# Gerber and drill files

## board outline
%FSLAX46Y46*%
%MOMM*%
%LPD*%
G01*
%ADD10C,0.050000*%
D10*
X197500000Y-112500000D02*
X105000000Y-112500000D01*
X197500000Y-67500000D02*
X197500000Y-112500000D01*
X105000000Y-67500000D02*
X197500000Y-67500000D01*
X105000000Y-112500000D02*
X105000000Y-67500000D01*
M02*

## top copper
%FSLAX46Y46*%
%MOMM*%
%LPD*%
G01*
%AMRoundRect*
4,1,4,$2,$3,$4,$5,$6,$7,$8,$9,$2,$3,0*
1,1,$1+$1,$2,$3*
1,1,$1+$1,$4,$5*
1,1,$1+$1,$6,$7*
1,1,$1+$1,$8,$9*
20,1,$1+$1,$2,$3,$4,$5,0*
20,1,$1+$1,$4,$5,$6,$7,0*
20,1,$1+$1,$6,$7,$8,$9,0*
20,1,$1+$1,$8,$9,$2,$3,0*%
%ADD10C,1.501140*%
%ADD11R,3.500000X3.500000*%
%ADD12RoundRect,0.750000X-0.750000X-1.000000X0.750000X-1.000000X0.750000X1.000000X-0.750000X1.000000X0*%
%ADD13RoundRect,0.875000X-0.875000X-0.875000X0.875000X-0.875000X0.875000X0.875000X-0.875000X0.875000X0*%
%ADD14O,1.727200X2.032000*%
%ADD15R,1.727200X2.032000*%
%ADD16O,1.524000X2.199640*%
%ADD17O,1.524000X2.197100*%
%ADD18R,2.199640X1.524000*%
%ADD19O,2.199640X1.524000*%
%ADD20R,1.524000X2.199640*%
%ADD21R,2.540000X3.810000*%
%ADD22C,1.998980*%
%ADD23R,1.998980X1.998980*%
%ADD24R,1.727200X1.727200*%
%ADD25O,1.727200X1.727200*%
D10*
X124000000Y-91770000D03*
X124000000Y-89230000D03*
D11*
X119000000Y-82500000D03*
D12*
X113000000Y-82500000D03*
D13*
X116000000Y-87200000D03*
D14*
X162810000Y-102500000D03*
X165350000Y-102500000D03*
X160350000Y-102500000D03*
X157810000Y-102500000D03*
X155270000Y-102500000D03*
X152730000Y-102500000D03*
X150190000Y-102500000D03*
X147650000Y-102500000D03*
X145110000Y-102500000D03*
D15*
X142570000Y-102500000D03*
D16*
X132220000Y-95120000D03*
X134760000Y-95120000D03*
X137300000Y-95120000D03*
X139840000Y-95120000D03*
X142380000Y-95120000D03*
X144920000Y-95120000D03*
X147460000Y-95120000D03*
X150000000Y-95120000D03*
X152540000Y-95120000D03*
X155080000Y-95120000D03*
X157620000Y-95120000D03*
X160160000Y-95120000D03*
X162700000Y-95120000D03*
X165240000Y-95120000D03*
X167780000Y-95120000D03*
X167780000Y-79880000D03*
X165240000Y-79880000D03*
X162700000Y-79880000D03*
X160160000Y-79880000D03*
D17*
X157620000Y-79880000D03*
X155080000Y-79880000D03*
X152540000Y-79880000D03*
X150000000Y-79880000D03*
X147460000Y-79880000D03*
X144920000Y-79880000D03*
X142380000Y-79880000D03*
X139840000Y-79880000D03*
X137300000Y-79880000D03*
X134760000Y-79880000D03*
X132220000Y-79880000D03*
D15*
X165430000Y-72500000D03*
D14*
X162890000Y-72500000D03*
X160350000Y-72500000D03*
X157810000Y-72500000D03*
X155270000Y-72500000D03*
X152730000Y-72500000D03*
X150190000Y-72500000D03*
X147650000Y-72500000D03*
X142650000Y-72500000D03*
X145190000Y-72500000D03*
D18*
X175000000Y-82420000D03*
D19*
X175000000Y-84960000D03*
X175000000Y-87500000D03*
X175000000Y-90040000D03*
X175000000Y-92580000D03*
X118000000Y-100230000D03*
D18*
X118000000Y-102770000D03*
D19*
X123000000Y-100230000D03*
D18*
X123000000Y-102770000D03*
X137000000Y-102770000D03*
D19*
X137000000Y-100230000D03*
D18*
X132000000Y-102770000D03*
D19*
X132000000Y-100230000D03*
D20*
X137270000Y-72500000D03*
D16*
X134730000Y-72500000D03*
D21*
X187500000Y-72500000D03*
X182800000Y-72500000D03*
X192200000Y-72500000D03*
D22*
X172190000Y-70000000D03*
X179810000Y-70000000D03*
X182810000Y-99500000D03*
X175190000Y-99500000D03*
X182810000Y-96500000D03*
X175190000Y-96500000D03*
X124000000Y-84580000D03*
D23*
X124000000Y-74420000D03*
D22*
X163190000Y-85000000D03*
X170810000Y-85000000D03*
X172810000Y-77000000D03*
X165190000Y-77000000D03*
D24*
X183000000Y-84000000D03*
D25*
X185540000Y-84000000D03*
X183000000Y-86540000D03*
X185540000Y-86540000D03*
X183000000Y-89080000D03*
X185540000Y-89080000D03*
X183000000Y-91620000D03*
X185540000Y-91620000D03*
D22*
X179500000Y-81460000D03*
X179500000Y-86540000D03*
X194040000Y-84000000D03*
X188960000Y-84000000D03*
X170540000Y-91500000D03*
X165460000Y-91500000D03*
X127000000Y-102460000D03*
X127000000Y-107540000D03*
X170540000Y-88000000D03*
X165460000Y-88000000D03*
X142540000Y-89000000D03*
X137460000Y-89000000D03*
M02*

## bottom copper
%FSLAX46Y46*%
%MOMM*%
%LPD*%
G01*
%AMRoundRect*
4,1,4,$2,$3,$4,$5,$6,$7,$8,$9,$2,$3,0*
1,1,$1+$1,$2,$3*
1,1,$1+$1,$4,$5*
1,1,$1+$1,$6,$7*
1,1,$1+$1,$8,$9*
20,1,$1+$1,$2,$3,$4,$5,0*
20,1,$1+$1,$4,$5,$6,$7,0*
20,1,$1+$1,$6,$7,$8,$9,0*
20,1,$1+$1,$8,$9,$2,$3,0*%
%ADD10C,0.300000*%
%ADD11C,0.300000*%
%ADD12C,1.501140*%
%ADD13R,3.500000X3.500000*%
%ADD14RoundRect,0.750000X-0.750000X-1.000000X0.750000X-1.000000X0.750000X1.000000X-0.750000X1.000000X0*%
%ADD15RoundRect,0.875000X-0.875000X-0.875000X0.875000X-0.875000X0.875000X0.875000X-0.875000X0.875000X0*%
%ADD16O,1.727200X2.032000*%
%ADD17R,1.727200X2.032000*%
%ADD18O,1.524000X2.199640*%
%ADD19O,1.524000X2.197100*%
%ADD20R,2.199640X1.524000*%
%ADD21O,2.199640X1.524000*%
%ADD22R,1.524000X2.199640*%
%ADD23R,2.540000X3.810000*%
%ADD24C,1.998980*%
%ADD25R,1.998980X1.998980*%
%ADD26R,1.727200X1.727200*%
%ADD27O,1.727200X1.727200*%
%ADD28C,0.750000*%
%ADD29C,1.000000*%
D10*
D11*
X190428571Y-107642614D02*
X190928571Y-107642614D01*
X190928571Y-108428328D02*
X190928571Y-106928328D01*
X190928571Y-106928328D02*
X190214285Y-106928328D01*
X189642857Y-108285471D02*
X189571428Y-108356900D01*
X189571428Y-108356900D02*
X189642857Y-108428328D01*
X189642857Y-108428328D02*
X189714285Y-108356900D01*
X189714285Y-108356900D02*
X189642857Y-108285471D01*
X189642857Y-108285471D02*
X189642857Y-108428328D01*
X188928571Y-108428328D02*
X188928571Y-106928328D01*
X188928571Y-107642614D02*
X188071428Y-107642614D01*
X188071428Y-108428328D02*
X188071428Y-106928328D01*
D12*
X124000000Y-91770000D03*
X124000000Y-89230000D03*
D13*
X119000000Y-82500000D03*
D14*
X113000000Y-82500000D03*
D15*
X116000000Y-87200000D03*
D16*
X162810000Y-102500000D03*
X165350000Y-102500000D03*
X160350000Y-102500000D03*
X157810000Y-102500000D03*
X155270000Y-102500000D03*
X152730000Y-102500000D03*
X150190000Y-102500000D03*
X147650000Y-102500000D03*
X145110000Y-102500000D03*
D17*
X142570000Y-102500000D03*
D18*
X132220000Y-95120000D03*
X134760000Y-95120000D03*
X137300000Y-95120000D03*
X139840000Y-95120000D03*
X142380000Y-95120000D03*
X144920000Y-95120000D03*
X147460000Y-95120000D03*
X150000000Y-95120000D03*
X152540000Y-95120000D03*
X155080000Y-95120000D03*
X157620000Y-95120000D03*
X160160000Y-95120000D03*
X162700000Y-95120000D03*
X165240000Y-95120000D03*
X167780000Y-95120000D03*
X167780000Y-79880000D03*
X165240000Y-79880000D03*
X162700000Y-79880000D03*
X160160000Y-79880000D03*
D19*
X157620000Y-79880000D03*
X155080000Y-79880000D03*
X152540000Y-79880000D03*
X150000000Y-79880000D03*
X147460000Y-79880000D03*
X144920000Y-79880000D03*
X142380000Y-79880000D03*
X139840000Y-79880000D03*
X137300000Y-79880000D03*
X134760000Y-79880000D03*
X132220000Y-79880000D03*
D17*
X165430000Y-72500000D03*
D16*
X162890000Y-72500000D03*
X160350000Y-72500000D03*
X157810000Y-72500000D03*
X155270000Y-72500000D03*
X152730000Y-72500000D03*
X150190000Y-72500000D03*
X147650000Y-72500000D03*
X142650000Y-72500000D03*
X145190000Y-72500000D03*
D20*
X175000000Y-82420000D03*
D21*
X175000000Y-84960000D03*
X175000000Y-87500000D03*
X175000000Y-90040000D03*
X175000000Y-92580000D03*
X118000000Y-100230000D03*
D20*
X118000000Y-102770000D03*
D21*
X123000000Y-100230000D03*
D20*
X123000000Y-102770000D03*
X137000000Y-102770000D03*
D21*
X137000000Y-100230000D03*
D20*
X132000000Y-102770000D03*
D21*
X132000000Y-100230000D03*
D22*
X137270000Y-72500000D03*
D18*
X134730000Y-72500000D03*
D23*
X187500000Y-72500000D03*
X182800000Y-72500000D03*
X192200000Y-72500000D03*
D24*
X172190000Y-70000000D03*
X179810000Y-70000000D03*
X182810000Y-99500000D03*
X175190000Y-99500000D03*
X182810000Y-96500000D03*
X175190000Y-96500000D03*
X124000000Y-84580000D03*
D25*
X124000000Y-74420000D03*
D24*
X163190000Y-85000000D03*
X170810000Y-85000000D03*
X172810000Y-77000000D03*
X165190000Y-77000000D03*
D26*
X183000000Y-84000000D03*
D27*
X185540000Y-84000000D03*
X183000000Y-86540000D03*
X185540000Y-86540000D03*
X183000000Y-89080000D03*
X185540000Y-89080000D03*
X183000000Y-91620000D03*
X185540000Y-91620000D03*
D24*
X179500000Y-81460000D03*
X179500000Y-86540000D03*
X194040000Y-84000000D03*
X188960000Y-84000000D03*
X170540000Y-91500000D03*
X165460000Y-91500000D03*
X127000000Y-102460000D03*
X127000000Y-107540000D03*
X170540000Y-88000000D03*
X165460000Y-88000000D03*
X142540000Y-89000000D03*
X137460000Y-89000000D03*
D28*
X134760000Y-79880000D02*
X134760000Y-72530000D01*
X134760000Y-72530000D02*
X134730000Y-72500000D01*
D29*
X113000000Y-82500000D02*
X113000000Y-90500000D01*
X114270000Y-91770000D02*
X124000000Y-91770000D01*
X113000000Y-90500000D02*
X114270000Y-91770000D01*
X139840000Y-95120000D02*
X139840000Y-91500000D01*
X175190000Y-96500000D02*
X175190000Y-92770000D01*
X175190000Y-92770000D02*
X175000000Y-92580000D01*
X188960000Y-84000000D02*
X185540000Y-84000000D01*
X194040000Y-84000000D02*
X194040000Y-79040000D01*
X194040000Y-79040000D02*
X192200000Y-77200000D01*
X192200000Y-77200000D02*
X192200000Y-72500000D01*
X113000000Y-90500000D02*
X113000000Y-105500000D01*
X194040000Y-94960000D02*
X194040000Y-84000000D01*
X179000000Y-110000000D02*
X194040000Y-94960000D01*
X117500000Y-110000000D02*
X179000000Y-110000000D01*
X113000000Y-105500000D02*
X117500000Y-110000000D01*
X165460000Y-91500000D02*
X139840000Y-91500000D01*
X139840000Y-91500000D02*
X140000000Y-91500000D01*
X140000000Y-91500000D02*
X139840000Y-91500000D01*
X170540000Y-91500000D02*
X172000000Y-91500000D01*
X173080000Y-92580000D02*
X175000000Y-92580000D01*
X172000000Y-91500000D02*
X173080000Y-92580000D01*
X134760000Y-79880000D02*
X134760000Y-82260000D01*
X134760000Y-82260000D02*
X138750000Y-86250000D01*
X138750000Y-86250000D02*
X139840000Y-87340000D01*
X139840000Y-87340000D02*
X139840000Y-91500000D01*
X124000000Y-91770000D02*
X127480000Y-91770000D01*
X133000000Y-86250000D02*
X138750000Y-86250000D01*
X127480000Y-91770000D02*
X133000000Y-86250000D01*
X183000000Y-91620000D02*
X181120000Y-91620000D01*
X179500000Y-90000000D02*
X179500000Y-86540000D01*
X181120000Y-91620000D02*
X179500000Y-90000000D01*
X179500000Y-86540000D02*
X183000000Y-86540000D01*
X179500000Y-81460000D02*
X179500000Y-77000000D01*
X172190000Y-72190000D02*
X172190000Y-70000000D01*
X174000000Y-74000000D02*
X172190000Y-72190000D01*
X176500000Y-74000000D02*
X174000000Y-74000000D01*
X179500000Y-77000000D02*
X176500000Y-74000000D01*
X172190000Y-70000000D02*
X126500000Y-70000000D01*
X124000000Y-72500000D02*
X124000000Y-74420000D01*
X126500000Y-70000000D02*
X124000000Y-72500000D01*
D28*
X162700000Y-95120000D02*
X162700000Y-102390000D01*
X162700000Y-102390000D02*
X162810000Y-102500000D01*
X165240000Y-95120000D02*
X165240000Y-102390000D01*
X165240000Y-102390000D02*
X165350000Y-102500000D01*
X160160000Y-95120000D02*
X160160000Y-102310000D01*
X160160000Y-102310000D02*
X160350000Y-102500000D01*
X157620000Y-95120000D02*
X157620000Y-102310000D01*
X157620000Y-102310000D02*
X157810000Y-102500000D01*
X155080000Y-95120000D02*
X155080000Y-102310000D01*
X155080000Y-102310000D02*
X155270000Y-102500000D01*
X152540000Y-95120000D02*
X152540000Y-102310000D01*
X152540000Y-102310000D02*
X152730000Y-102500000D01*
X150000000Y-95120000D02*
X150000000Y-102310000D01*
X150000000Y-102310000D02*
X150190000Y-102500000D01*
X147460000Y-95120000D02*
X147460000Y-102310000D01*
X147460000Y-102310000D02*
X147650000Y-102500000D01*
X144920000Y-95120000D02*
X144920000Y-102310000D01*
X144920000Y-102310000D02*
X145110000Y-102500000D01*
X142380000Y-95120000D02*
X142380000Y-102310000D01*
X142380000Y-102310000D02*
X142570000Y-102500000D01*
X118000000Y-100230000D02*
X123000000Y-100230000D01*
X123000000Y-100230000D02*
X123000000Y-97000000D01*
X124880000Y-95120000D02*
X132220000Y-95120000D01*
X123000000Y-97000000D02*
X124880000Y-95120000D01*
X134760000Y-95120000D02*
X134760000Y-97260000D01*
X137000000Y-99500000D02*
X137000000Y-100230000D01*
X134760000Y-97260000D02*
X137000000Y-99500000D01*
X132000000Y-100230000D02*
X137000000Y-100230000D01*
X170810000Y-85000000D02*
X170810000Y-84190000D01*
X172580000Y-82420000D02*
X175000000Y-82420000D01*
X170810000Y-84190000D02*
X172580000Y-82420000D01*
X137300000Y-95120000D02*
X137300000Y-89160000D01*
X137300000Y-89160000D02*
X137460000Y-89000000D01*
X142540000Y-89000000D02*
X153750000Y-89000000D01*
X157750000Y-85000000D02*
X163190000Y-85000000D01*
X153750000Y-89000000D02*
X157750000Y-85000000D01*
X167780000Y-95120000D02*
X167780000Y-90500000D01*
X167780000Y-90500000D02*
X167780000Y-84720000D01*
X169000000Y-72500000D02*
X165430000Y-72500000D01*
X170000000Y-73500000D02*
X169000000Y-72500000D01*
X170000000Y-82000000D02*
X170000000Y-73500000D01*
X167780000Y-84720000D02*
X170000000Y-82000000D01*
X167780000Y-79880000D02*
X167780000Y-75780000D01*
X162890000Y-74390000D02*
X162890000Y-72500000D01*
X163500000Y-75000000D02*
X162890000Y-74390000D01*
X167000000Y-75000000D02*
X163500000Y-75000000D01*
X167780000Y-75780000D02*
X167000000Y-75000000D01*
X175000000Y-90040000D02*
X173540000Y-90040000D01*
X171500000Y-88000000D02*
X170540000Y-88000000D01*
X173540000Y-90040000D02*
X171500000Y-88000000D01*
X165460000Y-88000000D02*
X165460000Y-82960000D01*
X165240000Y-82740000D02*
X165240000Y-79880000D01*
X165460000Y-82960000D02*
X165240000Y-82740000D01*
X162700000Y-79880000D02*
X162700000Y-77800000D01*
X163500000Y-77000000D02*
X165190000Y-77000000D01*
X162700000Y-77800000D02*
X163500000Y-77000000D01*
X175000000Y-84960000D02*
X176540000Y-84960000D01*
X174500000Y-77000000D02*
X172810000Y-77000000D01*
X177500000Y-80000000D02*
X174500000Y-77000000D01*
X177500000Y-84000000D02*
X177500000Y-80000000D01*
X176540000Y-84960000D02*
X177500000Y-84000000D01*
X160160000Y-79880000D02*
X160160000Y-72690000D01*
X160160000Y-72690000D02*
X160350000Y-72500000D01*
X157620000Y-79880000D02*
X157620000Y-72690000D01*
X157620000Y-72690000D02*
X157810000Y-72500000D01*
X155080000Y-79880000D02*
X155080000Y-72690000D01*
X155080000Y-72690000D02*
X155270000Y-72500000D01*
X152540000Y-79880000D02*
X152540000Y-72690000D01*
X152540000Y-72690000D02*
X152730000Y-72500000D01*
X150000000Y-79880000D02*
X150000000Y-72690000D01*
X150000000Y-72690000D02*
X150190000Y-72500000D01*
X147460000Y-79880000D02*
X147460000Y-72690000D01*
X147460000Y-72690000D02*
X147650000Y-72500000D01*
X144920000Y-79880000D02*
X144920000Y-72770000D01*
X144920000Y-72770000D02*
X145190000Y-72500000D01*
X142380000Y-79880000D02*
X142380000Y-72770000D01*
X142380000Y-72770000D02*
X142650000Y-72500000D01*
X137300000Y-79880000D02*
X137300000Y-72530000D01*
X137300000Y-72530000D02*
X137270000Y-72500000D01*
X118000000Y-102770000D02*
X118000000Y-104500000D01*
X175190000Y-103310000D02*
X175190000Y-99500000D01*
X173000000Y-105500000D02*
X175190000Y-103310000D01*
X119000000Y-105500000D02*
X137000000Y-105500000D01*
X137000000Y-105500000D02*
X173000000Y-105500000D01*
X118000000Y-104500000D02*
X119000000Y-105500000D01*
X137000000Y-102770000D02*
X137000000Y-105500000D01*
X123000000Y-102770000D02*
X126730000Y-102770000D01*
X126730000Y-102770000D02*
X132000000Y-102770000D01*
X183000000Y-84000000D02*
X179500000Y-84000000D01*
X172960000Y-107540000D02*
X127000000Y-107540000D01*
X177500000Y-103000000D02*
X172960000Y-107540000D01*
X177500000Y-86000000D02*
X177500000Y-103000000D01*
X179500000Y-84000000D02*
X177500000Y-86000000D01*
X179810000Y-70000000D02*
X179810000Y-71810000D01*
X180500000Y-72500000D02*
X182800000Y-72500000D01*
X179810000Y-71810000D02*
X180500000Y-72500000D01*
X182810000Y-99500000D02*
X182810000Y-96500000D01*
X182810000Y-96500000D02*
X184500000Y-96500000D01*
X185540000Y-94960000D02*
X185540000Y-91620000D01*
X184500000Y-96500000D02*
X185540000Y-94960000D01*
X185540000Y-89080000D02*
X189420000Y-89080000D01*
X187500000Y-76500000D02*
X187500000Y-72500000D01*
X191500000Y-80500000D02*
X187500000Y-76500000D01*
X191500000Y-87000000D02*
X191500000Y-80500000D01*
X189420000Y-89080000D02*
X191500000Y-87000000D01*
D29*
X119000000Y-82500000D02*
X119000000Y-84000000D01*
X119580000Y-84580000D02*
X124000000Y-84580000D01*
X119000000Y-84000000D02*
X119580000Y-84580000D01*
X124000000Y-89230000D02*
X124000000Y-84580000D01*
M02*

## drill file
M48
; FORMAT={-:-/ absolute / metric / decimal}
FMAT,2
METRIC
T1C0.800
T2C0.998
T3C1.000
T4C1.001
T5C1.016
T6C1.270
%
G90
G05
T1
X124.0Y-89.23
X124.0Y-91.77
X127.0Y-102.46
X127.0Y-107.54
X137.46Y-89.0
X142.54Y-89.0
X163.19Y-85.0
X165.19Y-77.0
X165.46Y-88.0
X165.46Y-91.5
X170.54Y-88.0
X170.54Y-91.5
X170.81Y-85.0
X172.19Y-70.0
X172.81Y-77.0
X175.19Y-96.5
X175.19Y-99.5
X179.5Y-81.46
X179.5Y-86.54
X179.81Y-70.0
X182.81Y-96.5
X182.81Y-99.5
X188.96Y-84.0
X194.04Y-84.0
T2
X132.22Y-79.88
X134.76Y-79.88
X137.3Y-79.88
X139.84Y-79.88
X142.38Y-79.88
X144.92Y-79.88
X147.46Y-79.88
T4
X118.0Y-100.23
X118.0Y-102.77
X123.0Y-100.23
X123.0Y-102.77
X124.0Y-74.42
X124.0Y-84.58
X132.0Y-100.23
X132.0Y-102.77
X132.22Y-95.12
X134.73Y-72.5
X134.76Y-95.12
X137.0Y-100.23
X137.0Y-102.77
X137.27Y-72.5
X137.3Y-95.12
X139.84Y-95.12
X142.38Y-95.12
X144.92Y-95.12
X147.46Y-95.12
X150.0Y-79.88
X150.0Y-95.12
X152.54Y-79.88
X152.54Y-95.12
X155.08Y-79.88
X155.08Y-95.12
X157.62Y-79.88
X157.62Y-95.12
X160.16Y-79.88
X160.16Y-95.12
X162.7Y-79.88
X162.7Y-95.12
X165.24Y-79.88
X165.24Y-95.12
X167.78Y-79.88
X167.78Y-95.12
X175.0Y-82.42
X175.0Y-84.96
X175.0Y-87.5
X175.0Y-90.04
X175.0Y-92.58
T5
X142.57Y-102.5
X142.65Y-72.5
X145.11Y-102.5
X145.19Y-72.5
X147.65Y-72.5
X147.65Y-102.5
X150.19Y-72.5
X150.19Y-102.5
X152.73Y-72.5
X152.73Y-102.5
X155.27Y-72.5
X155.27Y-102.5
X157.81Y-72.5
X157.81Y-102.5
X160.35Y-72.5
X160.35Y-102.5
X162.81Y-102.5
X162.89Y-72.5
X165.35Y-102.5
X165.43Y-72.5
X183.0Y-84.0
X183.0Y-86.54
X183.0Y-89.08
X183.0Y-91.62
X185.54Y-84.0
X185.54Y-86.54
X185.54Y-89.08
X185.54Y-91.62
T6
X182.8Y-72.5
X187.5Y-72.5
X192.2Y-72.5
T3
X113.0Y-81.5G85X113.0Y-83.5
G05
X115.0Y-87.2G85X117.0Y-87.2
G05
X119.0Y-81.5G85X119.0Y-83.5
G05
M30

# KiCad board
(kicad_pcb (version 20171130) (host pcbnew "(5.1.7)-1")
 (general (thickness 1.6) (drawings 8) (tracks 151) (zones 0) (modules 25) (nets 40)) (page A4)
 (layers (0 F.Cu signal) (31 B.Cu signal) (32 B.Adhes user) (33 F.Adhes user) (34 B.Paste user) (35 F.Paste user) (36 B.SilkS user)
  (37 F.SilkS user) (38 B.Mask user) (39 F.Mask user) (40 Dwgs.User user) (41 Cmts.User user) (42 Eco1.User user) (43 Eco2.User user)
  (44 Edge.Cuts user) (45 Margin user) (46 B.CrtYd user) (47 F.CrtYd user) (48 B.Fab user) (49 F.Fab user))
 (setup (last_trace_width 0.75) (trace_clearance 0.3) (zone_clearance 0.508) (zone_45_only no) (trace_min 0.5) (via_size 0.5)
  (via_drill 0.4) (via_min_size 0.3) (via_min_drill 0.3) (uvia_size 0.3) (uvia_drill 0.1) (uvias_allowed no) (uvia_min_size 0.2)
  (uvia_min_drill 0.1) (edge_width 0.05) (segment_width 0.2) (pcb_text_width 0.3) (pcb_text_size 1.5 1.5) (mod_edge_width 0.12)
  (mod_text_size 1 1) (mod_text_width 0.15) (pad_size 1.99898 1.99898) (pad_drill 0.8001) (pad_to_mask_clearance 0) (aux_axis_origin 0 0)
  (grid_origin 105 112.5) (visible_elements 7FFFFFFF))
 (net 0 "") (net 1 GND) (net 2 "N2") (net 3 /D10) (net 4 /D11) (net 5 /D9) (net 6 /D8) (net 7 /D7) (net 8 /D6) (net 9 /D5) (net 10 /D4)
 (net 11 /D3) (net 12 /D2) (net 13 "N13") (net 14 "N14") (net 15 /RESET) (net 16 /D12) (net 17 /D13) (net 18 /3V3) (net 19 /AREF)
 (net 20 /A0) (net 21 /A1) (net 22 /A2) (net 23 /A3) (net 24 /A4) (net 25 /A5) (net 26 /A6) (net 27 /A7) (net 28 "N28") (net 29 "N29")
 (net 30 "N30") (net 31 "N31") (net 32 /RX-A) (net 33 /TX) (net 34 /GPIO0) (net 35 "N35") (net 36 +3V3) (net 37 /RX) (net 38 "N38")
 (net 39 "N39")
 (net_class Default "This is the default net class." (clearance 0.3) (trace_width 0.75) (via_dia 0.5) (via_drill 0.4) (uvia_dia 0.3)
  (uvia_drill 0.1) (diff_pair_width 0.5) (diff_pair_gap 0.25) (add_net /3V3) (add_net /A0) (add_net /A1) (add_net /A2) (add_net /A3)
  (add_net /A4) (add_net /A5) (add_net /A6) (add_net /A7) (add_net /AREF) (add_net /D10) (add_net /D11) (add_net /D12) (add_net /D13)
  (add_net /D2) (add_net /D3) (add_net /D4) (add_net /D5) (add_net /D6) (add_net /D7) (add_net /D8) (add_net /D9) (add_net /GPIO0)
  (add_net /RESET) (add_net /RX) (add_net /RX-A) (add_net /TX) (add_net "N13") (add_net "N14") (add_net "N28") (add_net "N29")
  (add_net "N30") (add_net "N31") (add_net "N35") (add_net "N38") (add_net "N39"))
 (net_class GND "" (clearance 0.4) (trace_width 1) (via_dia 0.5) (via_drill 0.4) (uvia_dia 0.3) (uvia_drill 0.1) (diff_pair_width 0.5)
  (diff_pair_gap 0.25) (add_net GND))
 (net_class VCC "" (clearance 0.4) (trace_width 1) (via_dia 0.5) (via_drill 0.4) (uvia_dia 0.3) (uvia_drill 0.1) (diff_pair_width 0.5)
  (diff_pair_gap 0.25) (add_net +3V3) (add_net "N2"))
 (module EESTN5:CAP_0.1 (layer F.Cu) (at 124 90.5 90)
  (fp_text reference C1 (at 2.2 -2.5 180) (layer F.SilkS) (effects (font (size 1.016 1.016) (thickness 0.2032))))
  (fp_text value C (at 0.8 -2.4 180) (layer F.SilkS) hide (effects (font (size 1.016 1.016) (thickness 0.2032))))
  (pad 1 thru_hole circle (at -1.27 0 90) (size 1.50114 1.50114) (drill 0.8001) (layers *.Cu *.Mask F.SilkS) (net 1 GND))
  (pad 2 thru_hole circle (at 1.27 0 90) (size 1.50114 1.50114) (drill 0.8001) (layers *.Cu *.Mask F.SilkS) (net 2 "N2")))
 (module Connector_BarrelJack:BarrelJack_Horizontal (layer F.Cu) (at 119 82.5)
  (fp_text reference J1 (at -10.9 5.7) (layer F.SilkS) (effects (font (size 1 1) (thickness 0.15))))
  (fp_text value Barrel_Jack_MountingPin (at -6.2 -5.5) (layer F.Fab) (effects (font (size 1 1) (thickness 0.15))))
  (pad 1 thru_hole rect (at 0 0) (size 3.5 3.5) (drill oval 1 3) (layers *.Cu *.Mask) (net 2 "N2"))
  (pad 2 thru_hole roundrect (at -6 0) (size 3 3.5) (drill oval 1 3) (layers *.Cu *.Mask) (roundrect_rratio 0.25) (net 1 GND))
  (pad 3 thru_hole roundrect (at -3 4.7) (size 3.5 3.5) (drill oval 3 1) (layers *.Cu *.Mask) (roundrect_rratio 0.25)))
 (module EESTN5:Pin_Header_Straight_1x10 (layer F.Cu) (at 154 102.5 90)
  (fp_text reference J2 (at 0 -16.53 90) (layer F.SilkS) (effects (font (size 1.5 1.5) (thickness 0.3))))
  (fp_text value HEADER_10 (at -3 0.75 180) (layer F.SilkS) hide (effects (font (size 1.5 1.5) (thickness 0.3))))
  (pad 9 thru_hole oval (at 0 8.81 90) (size 2.032 1.7272) (drill 1.016) (layers *.Cu *.Mask F.SilkS) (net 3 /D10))
  (pad 10 thru_hole oval (at 0 11.35 90) (size 2.032 1.7272) (drill 1.016) (layers *.Cu *.Mask F.SilkS) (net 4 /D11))
  (pad 8 thru_hole oval (at 0 6.35 90) (size 2.032 1.7272) (drill 1.016) (layers *.Cu *.Mask F.SilkS) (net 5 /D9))
  (pad 7 thru_hole oval (at 0 3.81 90) (size 2.032 1.7272) (drill 1.016) (layers *.Cu *.Mask F.SilkS) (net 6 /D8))
  (pad 6 thru_hole oval (at 0 1.27 90) (size 2.032 1.7272) (drill 1.016) (layers *.Cu *.Mask F.SilkS) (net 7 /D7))
  (pad 5 thru_hole oval (at 0 -1.27 90) (size 2.032 1.7272) (drill 1.016) (layers *.Cu *.Mask F.SilkS) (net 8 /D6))
  (pad 4 thru_hole oval (at 0 -3.81 90) (size 2.032 1.7272) (drill 1.016) (layers *.Cu *.Mask F.SilkS) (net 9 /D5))
  (pad 3 thru_hole oval (at 0 -6.35 90) (size 2.032 1.7272) (drill 1.016) (layers *.Cu *.Mask F.SilkS) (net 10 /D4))
  (pad 2 thru_hole oval (at 0 -8.89 90) (size 2.032 1.7272) (drill 1.016) (layers *.Cu *.Mask F.SilkS) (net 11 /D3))
  (pad 1 thru_hole rect (at 0 -11.43 90) (size 2.032 1.7272) (drill 1.016) (layers *.Cu *.Mask F.SilkS) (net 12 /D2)))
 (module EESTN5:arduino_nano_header (layer F.Cu) (at 150 87.5)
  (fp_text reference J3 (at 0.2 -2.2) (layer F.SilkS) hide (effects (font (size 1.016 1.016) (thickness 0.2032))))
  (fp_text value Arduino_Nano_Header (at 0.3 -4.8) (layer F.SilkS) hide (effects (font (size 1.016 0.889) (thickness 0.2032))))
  (pad 1 thru_hole oval (at -17.78 7.62) (size 1.524 2.19964) (drill 1.00076) (layers *.Cu *.Mask F.SilkS) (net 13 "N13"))
  (pad 2 thru_hole oval (at -15.24 7.62) (size 1.524 2.19964) (drill 1.00076) (layers *.Cu *.Mask F.SilkS) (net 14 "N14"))
  (pad 3 thru_hole oval (at -12.7 7.62) (size 1.524 2.19964) (drill 1.00076) (layers *.Cu *.Mask F.SilkS) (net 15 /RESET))
  (pad 4 thru_hole oval (at -10.16 7.62) (size 1.524 2.19964) (drill 1.00076) (layers *.Cu *.Mask F.SilkS) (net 1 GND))
  (pad 5 thru_hole oval (at -7.62 7.62) (size 1.524 2.19964) (drill 1.00076) (layers *.Cu *.Mask F.SilkS) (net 12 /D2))
  (pad 6 thru_hole oval (at -5.08 7.62) (size 1.524 2.19964) (drill 1.00076) (layers *.Cu *.Mask F.SilkS) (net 11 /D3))
  (pad 7 thru_hole oval (at -2.54 7.62) (size 1.524 2.19964) (drill 1.00076) (layers *.Cu *.Mask F.SilkS) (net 10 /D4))
  (pad 8 thru_hole oval (at 0 7.62) (size 1.524 2.19964) (drill 1.00076) (layers *.Cu *.Mask F.SilkS) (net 9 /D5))
  (pad 9 thru_hole oval (at 2.54 7.62) (size 1.524 2.19964) (drill 1.00076) (layers *.Cu *.Mask F.SilkS) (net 8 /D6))
  (pad 10 thru_hole oval (at 5.08 7.62) (size 1.524 2.19964) (drill 1.00076) (layers *.Cu *.Mask F.SilkS) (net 7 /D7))
  (pad 11 thru_hole oval (at 7.62 7.62) (size 1.524 2.19964) (drill 1.00076) (layers *.Cu *.Mask F.SilkS) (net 6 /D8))
  (pad 12 thru_hole oval (at 10.16 7.62) (size 1.524 2.19964) (drill 1.00076) (layers *.Cu *.Mask F.SilkS) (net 5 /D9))
  (pad 13 thru_hole oval (at 12.7 7.62) (size 1.524 2.19964) (drill 1.00076) (layers *.Cu *.Mask F.SilkS) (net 3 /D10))
  (pad 14 thru_hole oval (at 15.24 7.62) (size 1.524 2.19964) (drill 1.00076) (layers *.Cu *.Mask F.SilkS) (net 4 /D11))
  (pad 15 thru_hole oval (at 17.78 7.62) (size 1.524 2.19964) (drill 1.00076) (layers *.Cu *.Mask F.SilkS) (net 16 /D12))
  (pad 16 thru_hole oval (at 17.78 -7.62) (size 1.524 2.19964) (drill 1.00076) (layers *.Cu *.Mask F.SilkS) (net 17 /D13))
  (pad 17 thru_hole oval (at 15.24 -7.62) (size 1.524 2.19964) (drill 1.00076) (layers *.Cu *.Mask F.SilkS) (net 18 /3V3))
  (pad 18 thru_hole oval (at 12.7 -7.62) (size 1.524 2.19964) (drill 1.00076) (layers *.Cu *.Mask F.SilkS) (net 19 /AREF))
  (pad 19 thru_hole oval (at 10.16 -7.62) (size 1.524 2.19964) (drill 1.00076) (layers *.Cu *.Mask F.SilkS) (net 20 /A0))
  (pad 20 thru_hole oval (at 7.62 -7.62) (size 1.524 2.1971) (drill 1.00076) (layers *.Cu *.Mask F.SilkS) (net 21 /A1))
  (pad 21 thru_hole oval (at 5.08 -7.62) (size 1.524 2.1971) (drill 1.00076) (layers *.Cu *.Mask F.SilkS) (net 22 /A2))
  (pad 22 thru_hole oval (at 2.54 -7.62) (size 1.524 2.1971) (drill 1.00076) (layers *.Cu *.Mask F.SilkS) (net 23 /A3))
  (pad 23 thru_hole oval (at 0 -7.62) (size 1.524 2.1971) (drill 1.00076) (layers *.Cu *.Mask F.SilkS) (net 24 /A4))
  (pad 24 thru_hole oval (at -2.54 -7.62) (size 1.524 2.1971) (drill 0.99822) (layers *.Cu *.Mask F.SilkS) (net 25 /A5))
  (pad 25 thru_hole oval (at -5.08 -7.62) (size 1.524 2.1971) (drill 0.99822) (layers *.Cu *.Mask F.SilkS) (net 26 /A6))
  (pad 26 thru_hole oval (at -7.62 -7.62) (size 1.524 2.1971) (drill 0.99822) (layers *.Cu *.Mask F.SilkS) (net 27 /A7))
  (pad 27 thru_hole oval (at -10.16 -7.62) (size 1.524 2.1971) (drill 0.99822) (layers *.Cu *.Mask F.SilkS) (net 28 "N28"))
  (pad 28 thru_hole oval (at -12.7 -7.62) (size 1.524 2.1971) (drill 0.99822) (layers *.Cu *.Mask F.SilkS) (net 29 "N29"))
  (pad 29 thru_hole oval (at -15.24 -7.62) (size 1.524 2.1971) (drill 0.99822) (layers *.Cu *.Mask F.SilkS) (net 1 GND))
  (pad 30 thru_hole oval (at -17.78 -7.62) (size 1.524 2.1971) (drill 0.99822) (layers *.Cu *.Mask F.SilkS) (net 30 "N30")))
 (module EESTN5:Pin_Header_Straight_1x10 (layer F.Cu) (at 154 72.5 270)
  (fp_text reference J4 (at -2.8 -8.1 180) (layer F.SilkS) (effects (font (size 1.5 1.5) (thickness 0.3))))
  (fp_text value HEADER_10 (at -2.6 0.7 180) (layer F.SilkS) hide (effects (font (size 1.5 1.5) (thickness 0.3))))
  (pad 1 thru_hole rect (at 0 -11.43 270) (size 2.032 1.7272) (drill 1.016) (layers *.Cu *.Mask F.SilkS) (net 16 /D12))
  (pad 2 thru_hole oval (at 0 -8.89 270) (size 2.032 1.7272) (drill 1.016) (layers *.Cu *.Mask F.SilkS) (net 17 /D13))
  (pad 3 thru_hole oval (at 0 -6.35 270) (size 2.032 1.7272) (drill 1.016) (layers *.Cu *.Mask F.SilkS) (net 20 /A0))
  (pad 4 thru_hole oval (at 0 -3.81 270) (size 2.032 1.7272) (drill 1.016) (layers *.Cu *.Mask F.SilkS) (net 21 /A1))
  (pad 5 thru_hole oval (at 0 -1.27 270) (size 2.032 1.7272) (drill 1.016) (layers *.Cu *.Mask F.SilkS) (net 22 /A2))
  (pad 6 thru_hole oval (at 0 1.27 270) (size 2.032 1.7272) (drill 1.016) (layers *.Cu *.Mask F.SilkS) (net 23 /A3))
  (pad 7 thru_hole oval (at 0 3.81 270) (size 2.032 1.7272) (drill 1.016) (layers *.Cu *.Mask F.SilkS) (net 24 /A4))
  (pad 8 thru_hole oval (at 0 6.35 270) (size 2.032 1.7272) (drill 1.016) (layers *.Cu *.Mask F.SilkS) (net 25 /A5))
  (pad 10 thru_hole oval (at 0 11.35 270) (size 2.032 1.7272) (drill 1.016) (layers *.Cu *.Mask F.SilkS) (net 27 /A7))
  (pad 9 thru_hole oval (at 0 8.81 270) (size 2.032 1.7272) (drill 1.016) (layers *.Cu *.Mask F.SilkS) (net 26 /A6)))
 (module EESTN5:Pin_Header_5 (layer F.Cu) (at 175 87.5 270)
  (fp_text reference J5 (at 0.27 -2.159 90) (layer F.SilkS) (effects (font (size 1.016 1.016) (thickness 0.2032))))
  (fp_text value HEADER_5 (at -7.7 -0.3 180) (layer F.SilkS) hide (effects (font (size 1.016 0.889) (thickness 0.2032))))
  (pad 1 thru_hole rect (at -5.08 0 270) (size 1.524 2.19964) (drill 1.00076) (layers *.Cu *.Mask F.SilkS) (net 15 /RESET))
  (pad 2 thru_hole oval (at -2.54 0 270) (size 1.524 2.19964) (drill 1.00076) (layers *.Cu *.Mask F.SilkS) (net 19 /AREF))
  (pad 3 thru_hole oval (at 0 0 270) (size 1.524 2.19964) (drill 1.00076) (layers *.Cu *.Mask F.SilkS) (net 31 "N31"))
  (pad 4 thru_hole oval (at 2.54 0 270) (size 1.524 2.19964) (drill 1.00076) (layers *.Cu *.Mask F.SilkS) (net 18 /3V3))
  (pad 5 thru_hole oval (at 5.08 0 270) (size 1.524 2.19964) (drill 1.00076) (layers *.Cu *.Mask F.SilkS) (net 1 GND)))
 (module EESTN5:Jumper (layer F.Cu) (at 118 101.5 90)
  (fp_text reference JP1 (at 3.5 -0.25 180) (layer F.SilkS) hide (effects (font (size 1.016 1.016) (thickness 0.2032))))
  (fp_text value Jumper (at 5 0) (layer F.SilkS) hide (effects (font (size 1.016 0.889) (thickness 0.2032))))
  (pad 2 thru_hole oval (at 1.27 0 90) (size 1.524 2.19964) (drill 1.00076) (layers *.Cu *.Mask F.SilkS) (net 13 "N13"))
  (pad 1 thru_hole rect (at -1.27 0 90) (size 1.524 2.19964) (drill 1.00076) (layers *.Cu *.Mask F.SilkS) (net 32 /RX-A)))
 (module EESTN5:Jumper (layer F.Cu) (at 123 101.5 90)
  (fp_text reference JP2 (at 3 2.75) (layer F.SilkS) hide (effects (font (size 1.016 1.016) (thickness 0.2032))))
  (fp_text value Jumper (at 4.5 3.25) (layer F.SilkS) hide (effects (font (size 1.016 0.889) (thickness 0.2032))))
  (pad 2 thru_hole oval (at 1.27 0 90) (size 1.524 2.19964) (drill 1.00076) (layers *.Cu *.Mask F.SilkS) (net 13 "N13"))
  (pad 1 thru_hole rect (at -1.27 0 90) (size 1.524 2.19964) (drill 1.00076) (layers *.Cu *.Mask F.SilkS) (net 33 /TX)))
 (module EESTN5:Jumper (layer F.Cu) (at 137 101.5 90)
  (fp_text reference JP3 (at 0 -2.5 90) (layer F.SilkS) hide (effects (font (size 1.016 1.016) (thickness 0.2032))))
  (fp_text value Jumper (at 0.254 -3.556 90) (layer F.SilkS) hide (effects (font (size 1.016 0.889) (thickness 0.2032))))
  (pad 1 thru_hole rect (at -1.27 0 90) (size 1.524 2.19964) (drill 1.00076) (layers *.Cu *.Mask F.SilkS) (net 32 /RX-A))
  (pad 2 thru_hole oval (at 1.27 0 90) (size 1.524 2.19964) (drill 1.00076) (layers *.Cu *.Mask F.SilkS) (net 14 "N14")))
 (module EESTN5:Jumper (layer F.Cu) (at 132 101.5 90)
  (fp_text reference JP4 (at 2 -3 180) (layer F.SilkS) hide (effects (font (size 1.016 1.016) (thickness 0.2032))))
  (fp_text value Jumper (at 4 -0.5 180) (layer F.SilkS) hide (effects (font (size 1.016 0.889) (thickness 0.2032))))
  (pad 1 thru_hole rect (at -1.27 0 90) (size 1.524 2.19964) (drill 1.00076) (layers *.Cu *.Mask F.SilkS) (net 33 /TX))
  (pad 2 thru_hole oval (at 1.27 0 90) (size 1.524 2.19964) (drill 1.00076) (layers *.Cu *.Mask F.SilkS) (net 14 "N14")))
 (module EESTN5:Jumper (layer F.Cu) (at 136 72.5 180)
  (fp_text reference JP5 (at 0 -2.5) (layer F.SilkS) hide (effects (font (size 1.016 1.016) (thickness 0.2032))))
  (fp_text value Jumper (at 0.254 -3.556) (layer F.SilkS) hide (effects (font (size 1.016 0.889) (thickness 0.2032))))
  (pad 1 thru_hole rect (at -1.27 0 180) (size 1.524 2.19964) (drill 1.00076) (layers *.Cu *.Mask F.SilkS) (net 29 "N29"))
  (pad 2 thru_hole oval (at 1.27 0 180) (size 1.524 2.19964) (drill 1.00076) (layers *.Cu *.Mask F.SilkS) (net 1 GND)))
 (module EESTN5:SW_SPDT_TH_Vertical (layer F.Cu) (at 187.5 72.5 90)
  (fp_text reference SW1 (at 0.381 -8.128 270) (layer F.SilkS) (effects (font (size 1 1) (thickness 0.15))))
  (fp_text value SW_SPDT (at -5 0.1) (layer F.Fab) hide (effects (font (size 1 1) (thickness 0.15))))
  (pad 2 thru_hole rect (at 0 0 90) (size 3.81 2.54) (drill 1.27) (layers *.Cu *.Mask) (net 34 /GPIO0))
  (pad 1 thru_hole rect (at 0 -4.7 90) (size 3.81 2.54) (drill 1.27) (layers *.Cu *.Mask) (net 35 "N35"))
  (pad 3 thru_hole rect (at 0 4.7 90) (size 3.81 2.54) (drill 1.27) (layers *.Cu *.Mask) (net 1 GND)))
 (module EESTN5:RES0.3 (layer F.Cu) (at 176 70) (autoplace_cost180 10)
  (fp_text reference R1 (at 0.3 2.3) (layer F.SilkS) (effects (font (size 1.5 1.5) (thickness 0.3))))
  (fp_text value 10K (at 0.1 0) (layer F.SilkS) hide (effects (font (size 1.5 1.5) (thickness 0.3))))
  (pad 1 thru_hole circle (at -3.81 0) (size 1.99898 1.99898) (drill 0.8001) (layers *.Cu *.Mask F.SilkS) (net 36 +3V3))
  (pad 2 thru_hole circle (at 3.81 0) (size 1.99898 1.99898) (drill 0.8001) (layers *.Cu *.Mask F.SilkS) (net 35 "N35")))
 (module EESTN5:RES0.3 (layer F.Cu) (at 179 99.5) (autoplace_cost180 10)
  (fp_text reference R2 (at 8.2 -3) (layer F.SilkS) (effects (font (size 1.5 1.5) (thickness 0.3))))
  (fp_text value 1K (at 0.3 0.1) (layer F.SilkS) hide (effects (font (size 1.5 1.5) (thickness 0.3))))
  (pad 2 thru_hole circle (at 3.81 0) (size 1.99898 1.99898) (drill 0.8001) (layers *.Cu *.Mask F.SilkS) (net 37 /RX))
  (pad 1 thru_hole circle (at -3.81 0) (size 1.99898 1.99898) (drill 0.8001) (layers *.Cu *.Mask F.SilkS) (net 32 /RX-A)))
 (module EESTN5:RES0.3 (layer F.Cu) (at 179 96.5 180) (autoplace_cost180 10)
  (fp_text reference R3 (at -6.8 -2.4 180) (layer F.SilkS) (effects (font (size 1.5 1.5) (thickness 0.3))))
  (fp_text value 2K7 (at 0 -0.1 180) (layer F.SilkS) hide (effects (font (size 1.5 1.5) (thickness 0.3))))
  (pad 1 thru_hole circle (at -3.81 0 180) (size 1.99898 1.99898) (drill 0.8001) (layers *.Cu *.Mask F.SilkS) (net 37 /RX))
  (pad 2 thru_hole circle (at 3.81 0 180) (size 1.99898 1.99898) (drill 0.8001) (layers *.Cu *.Mask F.SilkS) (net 1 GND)))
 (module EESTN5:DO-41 (layer F.Cu) (at 124 79.5 90)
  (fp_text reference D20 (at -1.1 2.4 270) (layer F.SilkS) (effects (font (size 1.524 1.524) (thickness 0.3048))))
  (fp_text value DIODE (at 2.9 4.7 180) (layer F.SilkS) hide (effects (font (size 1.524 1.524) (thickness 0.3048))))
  (pad 1 thru_hole circle (at -5.08 0 90) (size 1.99898 1.99898) (drill 1.00076) (layers *.Cu *.Mask F.SilkS) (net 2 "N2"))
  (pad 2 thru_hole rect (at 5.08 0 90) (size 1.99898 1.99898) (drill 1.00076) (layers *.Cu *.Mask F.SilkS) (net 36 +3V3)))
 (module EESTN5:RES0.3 (layer F.Cu) (at 167 85 180) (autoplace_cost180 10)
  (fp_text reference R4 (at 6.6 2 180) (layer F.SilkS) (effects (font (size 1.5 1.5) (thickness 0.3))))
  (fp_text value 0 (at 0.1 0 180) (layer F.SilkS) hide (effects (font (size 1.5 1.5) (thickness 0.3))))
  (pad 2 thru_hole circle (at 3.81 0 180) (size 1.99898 1.99898) (drill 0.8001) (layers *.Cu *.Mask F.SilkS) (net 15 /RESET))
  (pad 2 thru_hole circle (at -3.81 0 180) (size 1.99898 1.99898) (drill 0.8001) (layers *.Cu *.Mask F.SilkS) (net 15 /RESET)))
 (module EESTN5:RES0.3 (layer F.Cu) (at 169 77) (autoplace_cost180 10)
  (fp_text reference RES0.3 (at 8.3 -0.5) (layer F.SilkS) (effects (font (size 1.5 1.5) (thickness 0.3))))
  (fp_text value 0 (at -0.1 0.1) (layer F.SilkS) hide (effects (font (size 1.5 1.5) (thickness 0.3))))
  (pad 2 thru_hole circle (at 3.81 0) (size 1.99898 1.99898) (drill 0.8001) (layers *.Cu *.Mask F.SilkS) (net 19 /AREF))
  (pad 1 thru_hole circle (at -3.81 0) (size 1.99898 1.99898) (drill 0.8001) (layers *.Cu *.Mask F.SilkS) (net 19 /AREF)))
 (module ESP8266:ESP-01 (layer F.Cu) (at 183 84)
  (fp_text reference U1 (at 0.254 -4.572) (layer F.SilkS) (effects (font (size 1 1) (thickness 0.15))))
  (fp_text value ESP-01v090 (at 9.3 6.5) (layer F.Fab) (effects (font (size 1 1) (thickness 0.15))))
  (pad 1 thru_hole rect (at 0 0) (size 1.7272 1.7272) (drill 1.016) (layers *.Cu *.Mask F.SilkS) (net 33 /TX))
  (pad 2 thru_hole oval (at 2.54 0) (size 1.7272 1.7272) (drill 1.016) (layers *.Cu *.Mask F.SilkS) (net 1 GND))
  (pad 3 thru_hole oval (at 0 2.54) (size 1.7272 1.7272) (drill 1.016) (layers *.Cu *.Mask F.SilkS) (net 36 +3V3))
  (pad 4 thru_hole oval (at 2.54 2.54) (size 1.7272 1.7272) (drill 1.016) (layers *.Cu *.Mask F.SilkS) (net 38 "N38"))
  (pad 5 thru_hole oval (at 0 5.08) (size 1.7272 1.7272) (drill 1.016) (layers *.Cu *.Mask F.SilkS) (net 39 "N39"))
  (pad 6 thru_hole oval (at 2.54 5.08) (size 1.7272 1.7272) (drill 1.016) (layers *.Cu *.Mask F.SilkS) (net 34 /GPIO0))
  (pad 7 thru_hole oval (at 0 7.62) (size 1.7272 1.7272) (drill 1.016) (layers *.Cu *.Mask F.SilkS) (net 36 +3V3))
  (pad 8 thru_hole oval (at 2.54 7.62) (size 1.7272 1.7272) (drill 1.016) (layers *.Cu *.Mask F.SilkS) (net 37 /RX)))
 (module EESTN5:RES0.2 (layer F.Cu) (at 179.5 84 90)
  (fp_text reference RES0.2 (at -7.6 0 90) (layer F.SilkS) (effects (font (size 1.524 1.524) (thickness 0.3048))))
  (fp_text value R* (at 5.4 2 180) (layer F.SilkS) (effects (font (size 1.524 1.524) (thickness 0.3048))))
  (pad 2 thru_hole circle (at 2.54 0 90) (size 1.99898 1.99898) (drill 0.8001) (layers *.Cu *.Mask F.SilkS) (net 36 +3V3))
  (pad 1 thru_hole circle (at -2.54 0 90) (size 1.99898 1.99898) (drill 0.8001) (layers *.Cu *.Mask F.SilkS) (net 36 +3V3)))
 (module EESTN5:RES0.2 (layer F.Cu) (at 191.5 84)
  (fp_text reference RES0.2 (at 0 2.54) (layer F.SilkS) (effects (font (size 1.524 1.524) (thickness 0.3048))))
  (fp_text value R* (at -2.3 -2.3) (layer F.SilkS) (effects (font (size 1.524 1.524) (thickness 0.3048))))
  (pad 2 thru_hole circle (at 2.54 0) (size 1.99898 1.99898) (drill 0.8001) (layers *.Cu *.Mask F.SilkS) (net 1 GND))
  (pad 1 thru_hole circle (at -2.54 0) (size 1.99898 1.99898) (drill 0.8001) (layers *.Cu *.Mask F.SilkS) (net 1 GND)))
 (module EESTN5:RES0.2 (layer F.Cu) (at 168 91.5)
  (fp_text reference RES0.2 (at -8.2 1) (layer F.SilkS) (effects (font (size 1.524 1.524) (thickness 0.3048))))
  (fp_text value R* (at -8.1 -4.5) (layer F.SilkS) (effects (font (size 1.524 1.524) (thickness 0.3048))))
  (pad 2 thru_hole circle (at 2.54 0) (size 1.99898 1.99898) (drill 0.8001) (layers *.Cu *.Mask F.SilkS) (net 1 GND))
  (pad 1 thru_hole circle (at -2.54 0) (size 1.99898 1.99898) (drill 0.8001) (layers *.Cu *.Mask F.SilkS) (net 1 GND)))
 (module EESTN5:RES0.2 (layer F.Cu) (at 127 105 90)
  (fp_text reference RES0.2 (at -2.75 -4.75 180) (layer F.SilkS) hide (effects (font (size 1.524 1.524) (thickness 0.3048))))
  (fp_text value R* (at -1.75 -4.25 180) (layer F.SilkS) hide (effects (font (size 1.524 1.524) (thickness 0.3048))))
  (pad 2 thru_hole circle (at 2.54 0 90) (size 1.99898 1.99898) (drill 0.8001) (layers *.Cu *.Mask F.SilkS) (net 33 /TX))
  (pad 1 thru_hole circle (at -2.54 0 90) (size 1.99898 1.99898) (drill 0.8001) (layers *.Cu *.Mask F.SilkS) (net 33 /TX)))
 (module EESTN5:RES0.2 (layer F.Cu) (at 168 88)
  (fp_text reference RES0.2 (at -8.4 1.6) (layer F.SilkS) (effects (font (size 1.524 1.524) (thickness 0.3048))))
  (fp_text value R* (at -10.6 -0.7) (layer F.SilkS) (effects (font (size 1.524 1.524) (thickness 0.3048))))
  (pad 2 thru_hole circle (at 2.54 0) (size 1.99898 1.99898) (drill 0.8001) (layers *.Cu *.Mask F.SilkS) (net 18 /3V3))
  (pad 1 thru_hole circle (at -2.54 0) (size 1.99898 1.99898) (drill 0.8001) (layers *.Cu *.Mask F.SilkS) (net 18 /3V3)))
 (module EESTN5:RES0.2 (layer F.Cu) (at 140 89)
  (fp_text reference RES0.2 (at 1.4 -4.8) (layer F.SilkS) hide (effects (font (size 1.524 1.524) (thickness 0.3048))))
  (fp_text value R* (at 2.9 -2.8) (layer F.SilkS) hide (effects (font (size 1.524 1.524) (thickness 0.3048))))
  (pad 2 thru_hole circle (at 2.54 0) (size 1.99898 1.99898) (drill 0.8001) (layers *.Cu *.Mask F.SilkS) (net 15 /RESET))
  (pad 1 thru_hole circle (at -2.54 0) (size 1.99898 1.99898) (drill 0.8001) (layers *.Cu *.Mask F.SilkS) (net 15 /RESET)))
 (gr_line (start 197.5 112.5) (end 105 112.5) (angle 90) (layer Edge.Cuts) (width 0.05))
 (gr_line (start 197.5 67.5) (end 197.5 112.5) (angle 90) (layer Edge.Cuts) (width 0.05))
 (gr_line (start 105 67.5) (end 197.5 67.5) (angle 90) (layer Edge.Cuts) (width 0.05))
 (gr_line (start 105 112.5) (end 105 67.5) (angle 90) (layer Edge.Cuts) (width 0.05))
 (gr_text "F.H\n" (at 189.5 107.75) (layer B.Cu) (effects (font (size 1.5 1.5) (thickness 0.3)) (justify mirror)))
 (segment (start 134.76 79.88) (end 134.76 72.53) (width 0.75) (layer B.Cu) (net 1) (status C00000))
 (segment (start 134.76 72.53) (end 134.73 72.5) (width 0.75) (layer B.Cu) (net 1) (status C00000))
 (segment (start 113 82.5) (end 113 90.5) (width 1) (layer B.Cu) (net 1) (status 400000))
 (segment (start 114.27 91.77) (end 124 91.77) (width 1) (layer B.Cu) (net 1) (status 800000))
 (segment (start 113 90.5) (end 114.27 91.77) (width 1) (layer B.Cu) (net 1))
 (segment (start 139.84 95.12) (end 139.84 91.5) (width 1) (layer B.Cu) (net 1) (status 400000))
 (segment (start 175.19 96.5) (end 175.19 92.77) (width 1) (layer B.Cu) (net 1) (status C00000))
 (segment (start 175.19 92.77) (end 175 92.58) (width 1) (layer B.Cu) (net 1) (status C00000))
 (segment (start 188.96 84) (end 185.54 84) (width 1) (layer B.Cu) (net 1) (status C00000))
 (segment (start 194.04 84) (end 194.04 79.04) (width 1) (layer B.Cu) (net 1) (status 400000))
 (segment (start 194.04 79.04) (end 192.2 77.2) (width 1) (layer B.Cu) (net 1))
 (segment (start 192.2 77.2) (end 192.2 72.5) (width 1) (layer B.Cu) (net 1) (status 800000))
 (segment (start 113 90.5) (end 113 105.5) (width 1) (layer B.Cu) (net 1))
 (segment (start 194.04 94.96) (end 194.04 84) (width 1) (layer B.Cu) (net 1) (status 800000))
 (segment (start 179 110) (end 194.04 94.96) (width 1) (layer B.Cu) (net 1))
 (segment (start 117.5 110) (end 179 110) (width 1) (layer B.Cu) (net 1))
 (segment (start 113 105.5) (end 117.5 110) (width 1) (layer B.Cu) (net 1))
 (segment (start 165.46 91.5) (end 139.84 91.5) (width 1) (layer B.Cu) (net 1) (status 400000))
 (segment (start 139.84 91.5) (end 140 91.5) (width 1) (layer B.Cu) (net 1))
 (segment (start 140 91.5) (end 139.84 91.5) (width 1) (layer B.Cu) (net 1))
 (segment (start 170.54 91.5) (end 172 91.5) (width 1) (layer B.Cu) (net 1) (status 400000))
 (segment (start 173.08 92.58) (end 175 92.58) (width 1) (layer B.Cu) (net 1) (status 800000))
 (segment (start 172 91.5) (end 173.08 92.58) (width 1) (layer B.Cu) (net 1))
 (segment (start 134.76 79.88) (end 134.76 82.26) (width 1) (layer B.Cu) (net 1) (status 400000))
 (segment (start 134.76 82.26) (end 138.75 86.25) (width 1) (layer B.Cu) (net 1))
 (segment (start 138.75 86.25) (end 139.84 87.34) (width 1) (layer B.Cu) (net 1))
 (segment (start 139.84 87.34) (end 139.84 91.5) (width 1) (layer B.Cu) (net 1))
 (segment (start 124 91.77) (end 127.48 91.77) (width 1) (layer B.Cu) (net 1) (status 400000))
 (segment (start 133 86.25) (end 138.75 86.25) (width 1) (layer B.Cu) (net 1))
 (segment (start 127.48 91.77) (end 133 86.25) (width 1) (layer B.Cu) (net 1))
 (segment (start 183 91.62) (end 181.12 91.62) (width 1) (layer B.Cu) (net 36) (status 400000))
 (segment (start 179.5 90) (end 179.5 86.54) (width 1) (layer B.Cu) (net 36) (status 800000))
 (segment (start 181.12 91.62) (end 179.5 90) (width 1) (layer B.Cu) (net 36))
 (segment (start 179.5 86.54) (end 183 86.54) (width 1) (layer B.Cu) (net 36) (status C00000))
 (segment (start 179.5 81.46) (end 179.5 77) (width 1) (layer B.Cu) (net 36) (status 400000))
 (segment (start 172.19 72.19) (end 172.19 70) (width 1) (layer B.Cu) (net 36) (status 800000))
 (segment (start 174 74) (end 172.19 72.19) (width 1) (layer B.Cu) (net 36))
 (segment (start 176.5 74) (end 174 74) (width 1) (layer B.Cu) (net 36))
 (segment (start 179.5 77) (end 176.5 74) (width 1) (layer B.Cu) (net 36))
 (segment (start 172.19 70) (end 126.5 70) (width 1) (layer B.Cu) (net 36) (status 400000))
 (segment (start 124 72.5) (end 124 74.42) (width 1) (layer B.Cu) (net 36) (status 800000))
 (segment (start 126.5 70) (end 124 72.5) (width 1) (layer B.Cu) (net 36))
 (segment (start 162.7 95.12) (end 162.7 102.39) (width 0.75) (layer B.Cu) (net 3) (status C00000))
 (segment (start 162.7 102.39) (end 162.81 102.5) (width 0.75) (layer B.Cu) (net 3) (status C00000))
 (segment (start 165.24 95.12) (end 165.24 102.39) (width 0.75) (layer B.Cu) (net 4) (status C00000))
 (segment (start 165.24 102.39) (end 165.35 102.5) (width 0.75) (layer B.Cu) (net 4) (status C00000))
 (segment (start 160.16 95.12) (end 160.16 102.31) (width 0.75) (layer B.Cu) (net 5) (status C00000))
 (segment (start 160.16 102.31) (end 160.35 102.5) (width 0.75) (layer B.Cu) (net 5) (status C00000))
 (segment (start 157.62 95.12) (end 157.62 102.31) (width 0.75) (layer B.Cu) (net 6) (status C00000))
 (segment (start 157.62 102.31) (end 157.81 102.5) (width 0.75) (layer B.Cu) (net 6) (status C00000))
 (segment (start 155.08 95.12) (end 155.08 102.31) (width 0.75) (layer B.Cu) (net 7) (status C00000))
 (segment (start 155.08 102.31) (end 155.27 102.5) (width 0.75) (layer B.Cu) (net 7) (status C00000))
 (segment (start 152.54 95.12) (end 152.54 102.31) (width 0.75) (layer B.Cu) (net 8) (status C00000))
 (segment (start 152.54 102.31) (end 152.73 102.5) (width 0.75) (layer B.Cu) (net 8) (status C00000))
 (segment (start 150 95.12) (end 150 102.31) (width 0.75) (layer B.Cu) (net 9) (status C00000))
 (segment (start 150 102.31) (end 150.19 102.5) (width 0.75) (layer B.Cu) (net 9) (status C00000))
 (segment (start 147.46 95.12) (end 147.46 102.31) (width 0.75) (layer B.Cu) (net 10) (status C00000))
 (segment (start 147.46 102.31) (end 147.65 102.5) (width 0.75) (layer B.Cu) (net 10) (status C00000))
 (segment (start 144.92 95.12) (end 144.92 102.31) (width 0.75) (layer B.Cu) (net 11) (status C00000))
 (segment (start 144.92 102.31) (end 145.11 102.5) (width 0.75) (layer B.Cu) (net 11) (status C00000))
 (segment (start 142.38 95.12) (end 142.38 102.31) (width 0.75) (layer B.Cu) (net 12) (status C00000))
 (segment (start 142.38 102.31) (end 142.57 102.5) (width 0.75) (layer B.Cu) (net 12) (status C00000))
 (segment (start 118 100.23) (end 123 100.23) (width 0.75) (layer B.Cu) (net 13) (status C00000))
 (segment (start 123 100.23) (end 123 97) (width 0.75) (layer B.Cu) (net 13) (status 400000))
 (segment (start 124.88 95.12) (end 132.22 95.12) (width 0.75) (layer B.Cu) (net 13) (status 800000))
 (segment (start 123 97) (end 124.88 95.12) (width 0.75) (layer B.Cu) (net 13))
 (segment (start 134.76 95.12) (end 134.76 97.26) (width 0.75) (layer B.Cu) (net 14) (status 400000))
 (segment (start 137 99.5) (end 137 100.23) (width 0.75) (layer B.Cu) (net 14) (status C00000))
 (segment (start 134.76 97.26) (end 137 99.5) (width 0.75) (layer B.Cu) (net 14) (status 800000))
 (segment (start 132 100.23) (end 137 100.23) (width 0.75) (layer B.Cu) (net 14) (status C00000))
 (segment (start 170.81 85) (end 170.81 84.19) (width 0.75) (layer B.Cu) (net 15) (status C00000))
 (segment (start 172.58 82.42) (end 175 82.42) (width 0.75) (layer B.Cu) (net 15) (status 800000))
 (segment (start 170.81 84.19) (end 172.58 82.42) (width 0.75) (layer B.Cu) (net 15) (status 400000))
 (segment (start 137.3 95.12) (end 137.3 89.16) (width 0.75) (layer B.Cu) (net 15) (status C00000))
 (segment (start 137.3 89.16) (end 137.46 89) (width 0.75) (layer B.Cu) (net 15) (status C00000))
 (segment (start 142.54 89) (end 153.75 89) (width 0.75) (layer B.Cu) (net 15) (status 400000))
 (segment (start 157.75 85) (end 163.19 85) (width 0.75) (layer B.Cu) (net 15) (status 800000))
 (segment (start 153.75 89) (end 157.75 85) (width 0.75) (layer B.Cu) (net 15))
 (segment (start 167.78 95.12) (end 167.78 90.5) (width 0.75) (layer B.Cu) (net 16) (status 400000))
 (segment (start 167.78 90.5) (end 167.78 84.72) (width 0.75) (layer B.Cu) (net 16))
 (segment (start 169 72.5) (end 165.43 72.5) (width 0.75) (layer B.Cu) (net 16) (status 800000))
 (segment (start 170 73.5) (end 169 72.5) (width 0.75) (layer B.Cu) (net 16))
 (segment (start 170 82) (end 170 73.5) (width 0.75) (layer B.Cu) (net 16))
 (segment (start 167.78 84.72) (end 170 82) (width 0.75) (layer B.Cu) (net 16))
 (segment (start 167.78 79.88) (end 167.78 75.78) (width 0.75) (layer B.Cu) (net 17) (status 400000))
 (segment (start 162.89 74.39) (end 162.89 72.5) (width 0.75) (layer B.Cu) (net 17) (status 800000))
 (segment (start 163.5 75) (end 162.89 74.39) (width 0.75) (layer B.Cu) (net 17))
 (segment (start 167 75) (end 163.5 75) (width 0.75) (layer B.Cu) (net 17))
 (segment (start 167.78 75.78) (end 167 75) (width 0.75) (layer B.Cu) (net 17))
 (segment (start 175 90.04) (end 173.54 90.04) (width 0.75) (layer B.Cu) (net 18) (status 400000))
 (segment (start 171.5 88) (end 170.54 88) (width 0.75) (layer B.Cu) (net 18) (status C00000))
 (segment (start 173.54 90.04) (end 171.5 88) (width 0.75) (layer B.Cu) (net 18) (status 800000))
 (segment (start 165.46 88) (end 165.46 82.96) (width 0.75) (layer B.Cu) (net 18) (status 400000))
 (segment (start 165.24 82.74) (end 165.24 79.88) (width 0.75) (layer B.Cu) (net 18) (status 800000))
 (segment (start 165.46 82.96) (end 165.24 82.74) (width 0.75) (layer B.Cu) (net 18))
 (segment (start 162.7 79.88) (end 162.7 77.8) (width 0.75) (layer B.Cu) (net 19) (status 400000))
 (segment (start 163.5 77) (end 165.19 77) (width 0.75) (layer B.Cu) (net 19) (status 800000))
 (segment (start 162.7 77.8) (end 163.5 77) (width 0.75) (layer B.Cu) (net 19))
 (segment (start 175 84.96) (end 176.54 84.96) (width 0.75) (layer B.Cu) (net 19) (status 400000))
 (segment (start 174.5 77) (end 172.81 77) (width 0.75) (layer B.Cu) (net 19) (status 800000))
 (segment (start 177.5 80) (end 174.5 77) (width 0.75) (layer B.Cu) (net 19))
 (segment (start 177.5 84) (end 177.5 80) (width 0.75) (layer B.Cu) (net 19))
 (segment (start 176.54 84.96) (end 177.5 84) (width 0.75) (layer B.Cu) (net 19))
 (segment (start 160.16 79.88) (end 160.16 72.69) (width 0.75) (layer B.Cu) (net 20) (status C00000))
 (segment (start 160.16 72.69) (end 160.35 72.5) (width 0.75) (layer B.Cu) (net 20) (status C00000))
 (segment (start 157.62 79.88) (end 157.62 72.69) (width 0.75) (layer B.Cu) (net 21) (status C00000))
 (segment (start 157.62 72.69) (end 157.81 72.5) (width 0.75) (layer B.Cu) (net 21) (status C00000))
 (segment (start 155.08 79.88) (end 155.08 72.69) (width 0.75) (layer B.Cu) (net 22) (status C00000))
 (segment (start 155.08 72.69) (end 155.27 72.5) (width 0.75) (layer B.Cu) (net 22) (status C00000))
 (segment (start 152.54 79.88) (end 152.54 72.69) (width 0.75) (layer B.Cu) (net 23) (status C00000))
 (segment (start 152.54 72.69) (end 152.73 72.5) (width 0.75) (layer B.Cu) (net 23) (status C00000))
 (segment (start 150 79.88) (end 150 72.69) (width 0.75) (layer B.Cu) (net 24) (status C00000))
 (segment (start 150 72.69) (end 150.19 72.5) (width 0.75) (layer B.Cu) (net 24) (status C00000))
 (segment (start 147.46 79.88) (end 147.46 72.69) (width 0.75) (layer B.Cu) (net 25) (status C00000))
 (segment (start 147.46 72.69) (end 147.65 72.5) (width 0.75) (layer B.Cu) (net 25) (status C00000))
 (segment (start 144.92 79.88) (end 144.92 72.77) (width 0.75) (layer B.Cu) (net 26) (status C00000))
 (segment (start 144.92 72.77) (end 145.19 72.5) (width 0.75) (layer B.Cu) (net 26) (status C00000))
 (segment (start 142.38 79.88) (end 142.38 72.77) (width 0.75) (layer B.Cu) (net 27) (status C00000))
 (segment (start 142.38 72.77) (end 142.65 72.5) (width 0.75) (layer B.Cu) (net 27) (status C00000))
 (segment (start 137.3 79.88) (end 137.3 72.53) (width 0.75) (layer B.Cu) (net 29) (status C00000))
 (segment (start 137.3 72.53) (end 137.27 72.5) (width 0.75) (layer B.Cu) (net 29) (status C00000))
 (segment (start 118 102.77) (end 118 104.5) (width 0.75) (layer B.Cu) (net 32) (status 400000))
 (segment (start 175.19 103.31) (end 175.19 99.5) (width 0.75) (layer B.Cu) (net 32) (status 800000))
 (segment (start 173 105.5) (end 175.19 103.31) (width 0.75) (layer B.Cu) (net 32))
 (segment (start 119 105.5) (end 137 105.5) (width 0.75) (layer B.Cu) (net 32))
 (segment (start 137 105.5) (end 173 105.5) (width 0.75) (layer B.Cu) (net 32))
 (segment (start 118 104.5) (end 119 105.5) (width 0.75) (layer B.Cu) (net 32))
 (segment (start 137 102.77) (end 137 105.5) (width 0.75) (layer B.Cu) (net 32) (status 400000))
 (segment (start 123 102.77) (end 126.73 102.77) (width 0.75) (layer B.Cu) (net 33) (status 400000))
 (segment (start 126.73 102.77) (end 132 102.77) (width 0.75) (layer B.Cu) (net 33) (status 800000))
 (segment (start 183 84) (end 179.5 84) (width 0.75) (layer B.Cu) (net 33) (status 400000))
 (segment (start 172.96 107.54) (end 127 107.54) (width 0.75) (layer B.Cu) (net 33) (status 800000))
 (segment (start 177.5 103) (end 172.96 107.54) (width 0.75) (layer B.Cu) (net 33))
 (segment (start 177.5 86) (end 177.5 103) (width 0.75) (layer B.Cu) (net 33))
 (segment (start 179.5 84) (end 177.5 86) (width 0.75) (layer B.Cu) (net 33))
 (segment (start 179.81 70) (end 179.81 71.81) (width 0.75) (layer B.Cu) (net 35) (status 400000))
 (segment (start 180.5 72.5) (end 182.8 72.5) (width 0.75) (layer B.Cu) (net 35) (status 800000))
 (segment (start 179.81 71.81) (end 180.5 72.5) (width 0.75) (layer B.Cu) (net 35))
 (segment (start 182.81 99.5) (end 182.81 96.5) (width 0.75) (layer B.Cu) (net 37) (status C00000))
 (segment (start 182.81 96.5) (end 184.5 96.5) (width 0.75) (layer B.Cu) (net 37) (status 400000))
 (segment (start 185.54 94.96) (end 185.54 91.62) (width 0.75) (layer B.Cu) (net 37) (status 800000))
 (segment (start 184.5 96.5) (end 185.54 94.96) (width 0.75) (layer B.Cu) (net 37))
 (segment (start 185.54 89.08) (end 189.42 89.08) (width 0.75) (layer B.Cu) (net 34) (status 400000))
 (segment (start 187.5 76.5) (end 187.5 72.5) (width 0.75) (layer B.Cu) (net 34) (status 800000))
 (segment (start 191.5 80.5) (end 187.5 76.5) (width 0.75) (layer B.Cu) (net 34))
 (segment (start 191.5 87) (end 191.5 80.5) (width 0.75) (layer B.Cu) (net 34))
 (segment (start 189.42 89.08) (end 191.5 87) (width 0.75) (layer B.Cu) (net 34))
 (segment (start 119 82.5) (end 119 84) (width 1) (layer B.Cu) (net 2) (status C00000))
 (segment (start 119.58 84.58) (end 124 84.58) (width 1) (layer B.Cu) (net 2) (status 800000))
 (segment (start 119 84) (end 119.58 84.58) (width 1) (layer B.Cu) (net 2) (status 400000))
 (segment (start 124 89.23) (end 124 84.58) (width 1) (layer B.Cu) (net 2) (status C00000)))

